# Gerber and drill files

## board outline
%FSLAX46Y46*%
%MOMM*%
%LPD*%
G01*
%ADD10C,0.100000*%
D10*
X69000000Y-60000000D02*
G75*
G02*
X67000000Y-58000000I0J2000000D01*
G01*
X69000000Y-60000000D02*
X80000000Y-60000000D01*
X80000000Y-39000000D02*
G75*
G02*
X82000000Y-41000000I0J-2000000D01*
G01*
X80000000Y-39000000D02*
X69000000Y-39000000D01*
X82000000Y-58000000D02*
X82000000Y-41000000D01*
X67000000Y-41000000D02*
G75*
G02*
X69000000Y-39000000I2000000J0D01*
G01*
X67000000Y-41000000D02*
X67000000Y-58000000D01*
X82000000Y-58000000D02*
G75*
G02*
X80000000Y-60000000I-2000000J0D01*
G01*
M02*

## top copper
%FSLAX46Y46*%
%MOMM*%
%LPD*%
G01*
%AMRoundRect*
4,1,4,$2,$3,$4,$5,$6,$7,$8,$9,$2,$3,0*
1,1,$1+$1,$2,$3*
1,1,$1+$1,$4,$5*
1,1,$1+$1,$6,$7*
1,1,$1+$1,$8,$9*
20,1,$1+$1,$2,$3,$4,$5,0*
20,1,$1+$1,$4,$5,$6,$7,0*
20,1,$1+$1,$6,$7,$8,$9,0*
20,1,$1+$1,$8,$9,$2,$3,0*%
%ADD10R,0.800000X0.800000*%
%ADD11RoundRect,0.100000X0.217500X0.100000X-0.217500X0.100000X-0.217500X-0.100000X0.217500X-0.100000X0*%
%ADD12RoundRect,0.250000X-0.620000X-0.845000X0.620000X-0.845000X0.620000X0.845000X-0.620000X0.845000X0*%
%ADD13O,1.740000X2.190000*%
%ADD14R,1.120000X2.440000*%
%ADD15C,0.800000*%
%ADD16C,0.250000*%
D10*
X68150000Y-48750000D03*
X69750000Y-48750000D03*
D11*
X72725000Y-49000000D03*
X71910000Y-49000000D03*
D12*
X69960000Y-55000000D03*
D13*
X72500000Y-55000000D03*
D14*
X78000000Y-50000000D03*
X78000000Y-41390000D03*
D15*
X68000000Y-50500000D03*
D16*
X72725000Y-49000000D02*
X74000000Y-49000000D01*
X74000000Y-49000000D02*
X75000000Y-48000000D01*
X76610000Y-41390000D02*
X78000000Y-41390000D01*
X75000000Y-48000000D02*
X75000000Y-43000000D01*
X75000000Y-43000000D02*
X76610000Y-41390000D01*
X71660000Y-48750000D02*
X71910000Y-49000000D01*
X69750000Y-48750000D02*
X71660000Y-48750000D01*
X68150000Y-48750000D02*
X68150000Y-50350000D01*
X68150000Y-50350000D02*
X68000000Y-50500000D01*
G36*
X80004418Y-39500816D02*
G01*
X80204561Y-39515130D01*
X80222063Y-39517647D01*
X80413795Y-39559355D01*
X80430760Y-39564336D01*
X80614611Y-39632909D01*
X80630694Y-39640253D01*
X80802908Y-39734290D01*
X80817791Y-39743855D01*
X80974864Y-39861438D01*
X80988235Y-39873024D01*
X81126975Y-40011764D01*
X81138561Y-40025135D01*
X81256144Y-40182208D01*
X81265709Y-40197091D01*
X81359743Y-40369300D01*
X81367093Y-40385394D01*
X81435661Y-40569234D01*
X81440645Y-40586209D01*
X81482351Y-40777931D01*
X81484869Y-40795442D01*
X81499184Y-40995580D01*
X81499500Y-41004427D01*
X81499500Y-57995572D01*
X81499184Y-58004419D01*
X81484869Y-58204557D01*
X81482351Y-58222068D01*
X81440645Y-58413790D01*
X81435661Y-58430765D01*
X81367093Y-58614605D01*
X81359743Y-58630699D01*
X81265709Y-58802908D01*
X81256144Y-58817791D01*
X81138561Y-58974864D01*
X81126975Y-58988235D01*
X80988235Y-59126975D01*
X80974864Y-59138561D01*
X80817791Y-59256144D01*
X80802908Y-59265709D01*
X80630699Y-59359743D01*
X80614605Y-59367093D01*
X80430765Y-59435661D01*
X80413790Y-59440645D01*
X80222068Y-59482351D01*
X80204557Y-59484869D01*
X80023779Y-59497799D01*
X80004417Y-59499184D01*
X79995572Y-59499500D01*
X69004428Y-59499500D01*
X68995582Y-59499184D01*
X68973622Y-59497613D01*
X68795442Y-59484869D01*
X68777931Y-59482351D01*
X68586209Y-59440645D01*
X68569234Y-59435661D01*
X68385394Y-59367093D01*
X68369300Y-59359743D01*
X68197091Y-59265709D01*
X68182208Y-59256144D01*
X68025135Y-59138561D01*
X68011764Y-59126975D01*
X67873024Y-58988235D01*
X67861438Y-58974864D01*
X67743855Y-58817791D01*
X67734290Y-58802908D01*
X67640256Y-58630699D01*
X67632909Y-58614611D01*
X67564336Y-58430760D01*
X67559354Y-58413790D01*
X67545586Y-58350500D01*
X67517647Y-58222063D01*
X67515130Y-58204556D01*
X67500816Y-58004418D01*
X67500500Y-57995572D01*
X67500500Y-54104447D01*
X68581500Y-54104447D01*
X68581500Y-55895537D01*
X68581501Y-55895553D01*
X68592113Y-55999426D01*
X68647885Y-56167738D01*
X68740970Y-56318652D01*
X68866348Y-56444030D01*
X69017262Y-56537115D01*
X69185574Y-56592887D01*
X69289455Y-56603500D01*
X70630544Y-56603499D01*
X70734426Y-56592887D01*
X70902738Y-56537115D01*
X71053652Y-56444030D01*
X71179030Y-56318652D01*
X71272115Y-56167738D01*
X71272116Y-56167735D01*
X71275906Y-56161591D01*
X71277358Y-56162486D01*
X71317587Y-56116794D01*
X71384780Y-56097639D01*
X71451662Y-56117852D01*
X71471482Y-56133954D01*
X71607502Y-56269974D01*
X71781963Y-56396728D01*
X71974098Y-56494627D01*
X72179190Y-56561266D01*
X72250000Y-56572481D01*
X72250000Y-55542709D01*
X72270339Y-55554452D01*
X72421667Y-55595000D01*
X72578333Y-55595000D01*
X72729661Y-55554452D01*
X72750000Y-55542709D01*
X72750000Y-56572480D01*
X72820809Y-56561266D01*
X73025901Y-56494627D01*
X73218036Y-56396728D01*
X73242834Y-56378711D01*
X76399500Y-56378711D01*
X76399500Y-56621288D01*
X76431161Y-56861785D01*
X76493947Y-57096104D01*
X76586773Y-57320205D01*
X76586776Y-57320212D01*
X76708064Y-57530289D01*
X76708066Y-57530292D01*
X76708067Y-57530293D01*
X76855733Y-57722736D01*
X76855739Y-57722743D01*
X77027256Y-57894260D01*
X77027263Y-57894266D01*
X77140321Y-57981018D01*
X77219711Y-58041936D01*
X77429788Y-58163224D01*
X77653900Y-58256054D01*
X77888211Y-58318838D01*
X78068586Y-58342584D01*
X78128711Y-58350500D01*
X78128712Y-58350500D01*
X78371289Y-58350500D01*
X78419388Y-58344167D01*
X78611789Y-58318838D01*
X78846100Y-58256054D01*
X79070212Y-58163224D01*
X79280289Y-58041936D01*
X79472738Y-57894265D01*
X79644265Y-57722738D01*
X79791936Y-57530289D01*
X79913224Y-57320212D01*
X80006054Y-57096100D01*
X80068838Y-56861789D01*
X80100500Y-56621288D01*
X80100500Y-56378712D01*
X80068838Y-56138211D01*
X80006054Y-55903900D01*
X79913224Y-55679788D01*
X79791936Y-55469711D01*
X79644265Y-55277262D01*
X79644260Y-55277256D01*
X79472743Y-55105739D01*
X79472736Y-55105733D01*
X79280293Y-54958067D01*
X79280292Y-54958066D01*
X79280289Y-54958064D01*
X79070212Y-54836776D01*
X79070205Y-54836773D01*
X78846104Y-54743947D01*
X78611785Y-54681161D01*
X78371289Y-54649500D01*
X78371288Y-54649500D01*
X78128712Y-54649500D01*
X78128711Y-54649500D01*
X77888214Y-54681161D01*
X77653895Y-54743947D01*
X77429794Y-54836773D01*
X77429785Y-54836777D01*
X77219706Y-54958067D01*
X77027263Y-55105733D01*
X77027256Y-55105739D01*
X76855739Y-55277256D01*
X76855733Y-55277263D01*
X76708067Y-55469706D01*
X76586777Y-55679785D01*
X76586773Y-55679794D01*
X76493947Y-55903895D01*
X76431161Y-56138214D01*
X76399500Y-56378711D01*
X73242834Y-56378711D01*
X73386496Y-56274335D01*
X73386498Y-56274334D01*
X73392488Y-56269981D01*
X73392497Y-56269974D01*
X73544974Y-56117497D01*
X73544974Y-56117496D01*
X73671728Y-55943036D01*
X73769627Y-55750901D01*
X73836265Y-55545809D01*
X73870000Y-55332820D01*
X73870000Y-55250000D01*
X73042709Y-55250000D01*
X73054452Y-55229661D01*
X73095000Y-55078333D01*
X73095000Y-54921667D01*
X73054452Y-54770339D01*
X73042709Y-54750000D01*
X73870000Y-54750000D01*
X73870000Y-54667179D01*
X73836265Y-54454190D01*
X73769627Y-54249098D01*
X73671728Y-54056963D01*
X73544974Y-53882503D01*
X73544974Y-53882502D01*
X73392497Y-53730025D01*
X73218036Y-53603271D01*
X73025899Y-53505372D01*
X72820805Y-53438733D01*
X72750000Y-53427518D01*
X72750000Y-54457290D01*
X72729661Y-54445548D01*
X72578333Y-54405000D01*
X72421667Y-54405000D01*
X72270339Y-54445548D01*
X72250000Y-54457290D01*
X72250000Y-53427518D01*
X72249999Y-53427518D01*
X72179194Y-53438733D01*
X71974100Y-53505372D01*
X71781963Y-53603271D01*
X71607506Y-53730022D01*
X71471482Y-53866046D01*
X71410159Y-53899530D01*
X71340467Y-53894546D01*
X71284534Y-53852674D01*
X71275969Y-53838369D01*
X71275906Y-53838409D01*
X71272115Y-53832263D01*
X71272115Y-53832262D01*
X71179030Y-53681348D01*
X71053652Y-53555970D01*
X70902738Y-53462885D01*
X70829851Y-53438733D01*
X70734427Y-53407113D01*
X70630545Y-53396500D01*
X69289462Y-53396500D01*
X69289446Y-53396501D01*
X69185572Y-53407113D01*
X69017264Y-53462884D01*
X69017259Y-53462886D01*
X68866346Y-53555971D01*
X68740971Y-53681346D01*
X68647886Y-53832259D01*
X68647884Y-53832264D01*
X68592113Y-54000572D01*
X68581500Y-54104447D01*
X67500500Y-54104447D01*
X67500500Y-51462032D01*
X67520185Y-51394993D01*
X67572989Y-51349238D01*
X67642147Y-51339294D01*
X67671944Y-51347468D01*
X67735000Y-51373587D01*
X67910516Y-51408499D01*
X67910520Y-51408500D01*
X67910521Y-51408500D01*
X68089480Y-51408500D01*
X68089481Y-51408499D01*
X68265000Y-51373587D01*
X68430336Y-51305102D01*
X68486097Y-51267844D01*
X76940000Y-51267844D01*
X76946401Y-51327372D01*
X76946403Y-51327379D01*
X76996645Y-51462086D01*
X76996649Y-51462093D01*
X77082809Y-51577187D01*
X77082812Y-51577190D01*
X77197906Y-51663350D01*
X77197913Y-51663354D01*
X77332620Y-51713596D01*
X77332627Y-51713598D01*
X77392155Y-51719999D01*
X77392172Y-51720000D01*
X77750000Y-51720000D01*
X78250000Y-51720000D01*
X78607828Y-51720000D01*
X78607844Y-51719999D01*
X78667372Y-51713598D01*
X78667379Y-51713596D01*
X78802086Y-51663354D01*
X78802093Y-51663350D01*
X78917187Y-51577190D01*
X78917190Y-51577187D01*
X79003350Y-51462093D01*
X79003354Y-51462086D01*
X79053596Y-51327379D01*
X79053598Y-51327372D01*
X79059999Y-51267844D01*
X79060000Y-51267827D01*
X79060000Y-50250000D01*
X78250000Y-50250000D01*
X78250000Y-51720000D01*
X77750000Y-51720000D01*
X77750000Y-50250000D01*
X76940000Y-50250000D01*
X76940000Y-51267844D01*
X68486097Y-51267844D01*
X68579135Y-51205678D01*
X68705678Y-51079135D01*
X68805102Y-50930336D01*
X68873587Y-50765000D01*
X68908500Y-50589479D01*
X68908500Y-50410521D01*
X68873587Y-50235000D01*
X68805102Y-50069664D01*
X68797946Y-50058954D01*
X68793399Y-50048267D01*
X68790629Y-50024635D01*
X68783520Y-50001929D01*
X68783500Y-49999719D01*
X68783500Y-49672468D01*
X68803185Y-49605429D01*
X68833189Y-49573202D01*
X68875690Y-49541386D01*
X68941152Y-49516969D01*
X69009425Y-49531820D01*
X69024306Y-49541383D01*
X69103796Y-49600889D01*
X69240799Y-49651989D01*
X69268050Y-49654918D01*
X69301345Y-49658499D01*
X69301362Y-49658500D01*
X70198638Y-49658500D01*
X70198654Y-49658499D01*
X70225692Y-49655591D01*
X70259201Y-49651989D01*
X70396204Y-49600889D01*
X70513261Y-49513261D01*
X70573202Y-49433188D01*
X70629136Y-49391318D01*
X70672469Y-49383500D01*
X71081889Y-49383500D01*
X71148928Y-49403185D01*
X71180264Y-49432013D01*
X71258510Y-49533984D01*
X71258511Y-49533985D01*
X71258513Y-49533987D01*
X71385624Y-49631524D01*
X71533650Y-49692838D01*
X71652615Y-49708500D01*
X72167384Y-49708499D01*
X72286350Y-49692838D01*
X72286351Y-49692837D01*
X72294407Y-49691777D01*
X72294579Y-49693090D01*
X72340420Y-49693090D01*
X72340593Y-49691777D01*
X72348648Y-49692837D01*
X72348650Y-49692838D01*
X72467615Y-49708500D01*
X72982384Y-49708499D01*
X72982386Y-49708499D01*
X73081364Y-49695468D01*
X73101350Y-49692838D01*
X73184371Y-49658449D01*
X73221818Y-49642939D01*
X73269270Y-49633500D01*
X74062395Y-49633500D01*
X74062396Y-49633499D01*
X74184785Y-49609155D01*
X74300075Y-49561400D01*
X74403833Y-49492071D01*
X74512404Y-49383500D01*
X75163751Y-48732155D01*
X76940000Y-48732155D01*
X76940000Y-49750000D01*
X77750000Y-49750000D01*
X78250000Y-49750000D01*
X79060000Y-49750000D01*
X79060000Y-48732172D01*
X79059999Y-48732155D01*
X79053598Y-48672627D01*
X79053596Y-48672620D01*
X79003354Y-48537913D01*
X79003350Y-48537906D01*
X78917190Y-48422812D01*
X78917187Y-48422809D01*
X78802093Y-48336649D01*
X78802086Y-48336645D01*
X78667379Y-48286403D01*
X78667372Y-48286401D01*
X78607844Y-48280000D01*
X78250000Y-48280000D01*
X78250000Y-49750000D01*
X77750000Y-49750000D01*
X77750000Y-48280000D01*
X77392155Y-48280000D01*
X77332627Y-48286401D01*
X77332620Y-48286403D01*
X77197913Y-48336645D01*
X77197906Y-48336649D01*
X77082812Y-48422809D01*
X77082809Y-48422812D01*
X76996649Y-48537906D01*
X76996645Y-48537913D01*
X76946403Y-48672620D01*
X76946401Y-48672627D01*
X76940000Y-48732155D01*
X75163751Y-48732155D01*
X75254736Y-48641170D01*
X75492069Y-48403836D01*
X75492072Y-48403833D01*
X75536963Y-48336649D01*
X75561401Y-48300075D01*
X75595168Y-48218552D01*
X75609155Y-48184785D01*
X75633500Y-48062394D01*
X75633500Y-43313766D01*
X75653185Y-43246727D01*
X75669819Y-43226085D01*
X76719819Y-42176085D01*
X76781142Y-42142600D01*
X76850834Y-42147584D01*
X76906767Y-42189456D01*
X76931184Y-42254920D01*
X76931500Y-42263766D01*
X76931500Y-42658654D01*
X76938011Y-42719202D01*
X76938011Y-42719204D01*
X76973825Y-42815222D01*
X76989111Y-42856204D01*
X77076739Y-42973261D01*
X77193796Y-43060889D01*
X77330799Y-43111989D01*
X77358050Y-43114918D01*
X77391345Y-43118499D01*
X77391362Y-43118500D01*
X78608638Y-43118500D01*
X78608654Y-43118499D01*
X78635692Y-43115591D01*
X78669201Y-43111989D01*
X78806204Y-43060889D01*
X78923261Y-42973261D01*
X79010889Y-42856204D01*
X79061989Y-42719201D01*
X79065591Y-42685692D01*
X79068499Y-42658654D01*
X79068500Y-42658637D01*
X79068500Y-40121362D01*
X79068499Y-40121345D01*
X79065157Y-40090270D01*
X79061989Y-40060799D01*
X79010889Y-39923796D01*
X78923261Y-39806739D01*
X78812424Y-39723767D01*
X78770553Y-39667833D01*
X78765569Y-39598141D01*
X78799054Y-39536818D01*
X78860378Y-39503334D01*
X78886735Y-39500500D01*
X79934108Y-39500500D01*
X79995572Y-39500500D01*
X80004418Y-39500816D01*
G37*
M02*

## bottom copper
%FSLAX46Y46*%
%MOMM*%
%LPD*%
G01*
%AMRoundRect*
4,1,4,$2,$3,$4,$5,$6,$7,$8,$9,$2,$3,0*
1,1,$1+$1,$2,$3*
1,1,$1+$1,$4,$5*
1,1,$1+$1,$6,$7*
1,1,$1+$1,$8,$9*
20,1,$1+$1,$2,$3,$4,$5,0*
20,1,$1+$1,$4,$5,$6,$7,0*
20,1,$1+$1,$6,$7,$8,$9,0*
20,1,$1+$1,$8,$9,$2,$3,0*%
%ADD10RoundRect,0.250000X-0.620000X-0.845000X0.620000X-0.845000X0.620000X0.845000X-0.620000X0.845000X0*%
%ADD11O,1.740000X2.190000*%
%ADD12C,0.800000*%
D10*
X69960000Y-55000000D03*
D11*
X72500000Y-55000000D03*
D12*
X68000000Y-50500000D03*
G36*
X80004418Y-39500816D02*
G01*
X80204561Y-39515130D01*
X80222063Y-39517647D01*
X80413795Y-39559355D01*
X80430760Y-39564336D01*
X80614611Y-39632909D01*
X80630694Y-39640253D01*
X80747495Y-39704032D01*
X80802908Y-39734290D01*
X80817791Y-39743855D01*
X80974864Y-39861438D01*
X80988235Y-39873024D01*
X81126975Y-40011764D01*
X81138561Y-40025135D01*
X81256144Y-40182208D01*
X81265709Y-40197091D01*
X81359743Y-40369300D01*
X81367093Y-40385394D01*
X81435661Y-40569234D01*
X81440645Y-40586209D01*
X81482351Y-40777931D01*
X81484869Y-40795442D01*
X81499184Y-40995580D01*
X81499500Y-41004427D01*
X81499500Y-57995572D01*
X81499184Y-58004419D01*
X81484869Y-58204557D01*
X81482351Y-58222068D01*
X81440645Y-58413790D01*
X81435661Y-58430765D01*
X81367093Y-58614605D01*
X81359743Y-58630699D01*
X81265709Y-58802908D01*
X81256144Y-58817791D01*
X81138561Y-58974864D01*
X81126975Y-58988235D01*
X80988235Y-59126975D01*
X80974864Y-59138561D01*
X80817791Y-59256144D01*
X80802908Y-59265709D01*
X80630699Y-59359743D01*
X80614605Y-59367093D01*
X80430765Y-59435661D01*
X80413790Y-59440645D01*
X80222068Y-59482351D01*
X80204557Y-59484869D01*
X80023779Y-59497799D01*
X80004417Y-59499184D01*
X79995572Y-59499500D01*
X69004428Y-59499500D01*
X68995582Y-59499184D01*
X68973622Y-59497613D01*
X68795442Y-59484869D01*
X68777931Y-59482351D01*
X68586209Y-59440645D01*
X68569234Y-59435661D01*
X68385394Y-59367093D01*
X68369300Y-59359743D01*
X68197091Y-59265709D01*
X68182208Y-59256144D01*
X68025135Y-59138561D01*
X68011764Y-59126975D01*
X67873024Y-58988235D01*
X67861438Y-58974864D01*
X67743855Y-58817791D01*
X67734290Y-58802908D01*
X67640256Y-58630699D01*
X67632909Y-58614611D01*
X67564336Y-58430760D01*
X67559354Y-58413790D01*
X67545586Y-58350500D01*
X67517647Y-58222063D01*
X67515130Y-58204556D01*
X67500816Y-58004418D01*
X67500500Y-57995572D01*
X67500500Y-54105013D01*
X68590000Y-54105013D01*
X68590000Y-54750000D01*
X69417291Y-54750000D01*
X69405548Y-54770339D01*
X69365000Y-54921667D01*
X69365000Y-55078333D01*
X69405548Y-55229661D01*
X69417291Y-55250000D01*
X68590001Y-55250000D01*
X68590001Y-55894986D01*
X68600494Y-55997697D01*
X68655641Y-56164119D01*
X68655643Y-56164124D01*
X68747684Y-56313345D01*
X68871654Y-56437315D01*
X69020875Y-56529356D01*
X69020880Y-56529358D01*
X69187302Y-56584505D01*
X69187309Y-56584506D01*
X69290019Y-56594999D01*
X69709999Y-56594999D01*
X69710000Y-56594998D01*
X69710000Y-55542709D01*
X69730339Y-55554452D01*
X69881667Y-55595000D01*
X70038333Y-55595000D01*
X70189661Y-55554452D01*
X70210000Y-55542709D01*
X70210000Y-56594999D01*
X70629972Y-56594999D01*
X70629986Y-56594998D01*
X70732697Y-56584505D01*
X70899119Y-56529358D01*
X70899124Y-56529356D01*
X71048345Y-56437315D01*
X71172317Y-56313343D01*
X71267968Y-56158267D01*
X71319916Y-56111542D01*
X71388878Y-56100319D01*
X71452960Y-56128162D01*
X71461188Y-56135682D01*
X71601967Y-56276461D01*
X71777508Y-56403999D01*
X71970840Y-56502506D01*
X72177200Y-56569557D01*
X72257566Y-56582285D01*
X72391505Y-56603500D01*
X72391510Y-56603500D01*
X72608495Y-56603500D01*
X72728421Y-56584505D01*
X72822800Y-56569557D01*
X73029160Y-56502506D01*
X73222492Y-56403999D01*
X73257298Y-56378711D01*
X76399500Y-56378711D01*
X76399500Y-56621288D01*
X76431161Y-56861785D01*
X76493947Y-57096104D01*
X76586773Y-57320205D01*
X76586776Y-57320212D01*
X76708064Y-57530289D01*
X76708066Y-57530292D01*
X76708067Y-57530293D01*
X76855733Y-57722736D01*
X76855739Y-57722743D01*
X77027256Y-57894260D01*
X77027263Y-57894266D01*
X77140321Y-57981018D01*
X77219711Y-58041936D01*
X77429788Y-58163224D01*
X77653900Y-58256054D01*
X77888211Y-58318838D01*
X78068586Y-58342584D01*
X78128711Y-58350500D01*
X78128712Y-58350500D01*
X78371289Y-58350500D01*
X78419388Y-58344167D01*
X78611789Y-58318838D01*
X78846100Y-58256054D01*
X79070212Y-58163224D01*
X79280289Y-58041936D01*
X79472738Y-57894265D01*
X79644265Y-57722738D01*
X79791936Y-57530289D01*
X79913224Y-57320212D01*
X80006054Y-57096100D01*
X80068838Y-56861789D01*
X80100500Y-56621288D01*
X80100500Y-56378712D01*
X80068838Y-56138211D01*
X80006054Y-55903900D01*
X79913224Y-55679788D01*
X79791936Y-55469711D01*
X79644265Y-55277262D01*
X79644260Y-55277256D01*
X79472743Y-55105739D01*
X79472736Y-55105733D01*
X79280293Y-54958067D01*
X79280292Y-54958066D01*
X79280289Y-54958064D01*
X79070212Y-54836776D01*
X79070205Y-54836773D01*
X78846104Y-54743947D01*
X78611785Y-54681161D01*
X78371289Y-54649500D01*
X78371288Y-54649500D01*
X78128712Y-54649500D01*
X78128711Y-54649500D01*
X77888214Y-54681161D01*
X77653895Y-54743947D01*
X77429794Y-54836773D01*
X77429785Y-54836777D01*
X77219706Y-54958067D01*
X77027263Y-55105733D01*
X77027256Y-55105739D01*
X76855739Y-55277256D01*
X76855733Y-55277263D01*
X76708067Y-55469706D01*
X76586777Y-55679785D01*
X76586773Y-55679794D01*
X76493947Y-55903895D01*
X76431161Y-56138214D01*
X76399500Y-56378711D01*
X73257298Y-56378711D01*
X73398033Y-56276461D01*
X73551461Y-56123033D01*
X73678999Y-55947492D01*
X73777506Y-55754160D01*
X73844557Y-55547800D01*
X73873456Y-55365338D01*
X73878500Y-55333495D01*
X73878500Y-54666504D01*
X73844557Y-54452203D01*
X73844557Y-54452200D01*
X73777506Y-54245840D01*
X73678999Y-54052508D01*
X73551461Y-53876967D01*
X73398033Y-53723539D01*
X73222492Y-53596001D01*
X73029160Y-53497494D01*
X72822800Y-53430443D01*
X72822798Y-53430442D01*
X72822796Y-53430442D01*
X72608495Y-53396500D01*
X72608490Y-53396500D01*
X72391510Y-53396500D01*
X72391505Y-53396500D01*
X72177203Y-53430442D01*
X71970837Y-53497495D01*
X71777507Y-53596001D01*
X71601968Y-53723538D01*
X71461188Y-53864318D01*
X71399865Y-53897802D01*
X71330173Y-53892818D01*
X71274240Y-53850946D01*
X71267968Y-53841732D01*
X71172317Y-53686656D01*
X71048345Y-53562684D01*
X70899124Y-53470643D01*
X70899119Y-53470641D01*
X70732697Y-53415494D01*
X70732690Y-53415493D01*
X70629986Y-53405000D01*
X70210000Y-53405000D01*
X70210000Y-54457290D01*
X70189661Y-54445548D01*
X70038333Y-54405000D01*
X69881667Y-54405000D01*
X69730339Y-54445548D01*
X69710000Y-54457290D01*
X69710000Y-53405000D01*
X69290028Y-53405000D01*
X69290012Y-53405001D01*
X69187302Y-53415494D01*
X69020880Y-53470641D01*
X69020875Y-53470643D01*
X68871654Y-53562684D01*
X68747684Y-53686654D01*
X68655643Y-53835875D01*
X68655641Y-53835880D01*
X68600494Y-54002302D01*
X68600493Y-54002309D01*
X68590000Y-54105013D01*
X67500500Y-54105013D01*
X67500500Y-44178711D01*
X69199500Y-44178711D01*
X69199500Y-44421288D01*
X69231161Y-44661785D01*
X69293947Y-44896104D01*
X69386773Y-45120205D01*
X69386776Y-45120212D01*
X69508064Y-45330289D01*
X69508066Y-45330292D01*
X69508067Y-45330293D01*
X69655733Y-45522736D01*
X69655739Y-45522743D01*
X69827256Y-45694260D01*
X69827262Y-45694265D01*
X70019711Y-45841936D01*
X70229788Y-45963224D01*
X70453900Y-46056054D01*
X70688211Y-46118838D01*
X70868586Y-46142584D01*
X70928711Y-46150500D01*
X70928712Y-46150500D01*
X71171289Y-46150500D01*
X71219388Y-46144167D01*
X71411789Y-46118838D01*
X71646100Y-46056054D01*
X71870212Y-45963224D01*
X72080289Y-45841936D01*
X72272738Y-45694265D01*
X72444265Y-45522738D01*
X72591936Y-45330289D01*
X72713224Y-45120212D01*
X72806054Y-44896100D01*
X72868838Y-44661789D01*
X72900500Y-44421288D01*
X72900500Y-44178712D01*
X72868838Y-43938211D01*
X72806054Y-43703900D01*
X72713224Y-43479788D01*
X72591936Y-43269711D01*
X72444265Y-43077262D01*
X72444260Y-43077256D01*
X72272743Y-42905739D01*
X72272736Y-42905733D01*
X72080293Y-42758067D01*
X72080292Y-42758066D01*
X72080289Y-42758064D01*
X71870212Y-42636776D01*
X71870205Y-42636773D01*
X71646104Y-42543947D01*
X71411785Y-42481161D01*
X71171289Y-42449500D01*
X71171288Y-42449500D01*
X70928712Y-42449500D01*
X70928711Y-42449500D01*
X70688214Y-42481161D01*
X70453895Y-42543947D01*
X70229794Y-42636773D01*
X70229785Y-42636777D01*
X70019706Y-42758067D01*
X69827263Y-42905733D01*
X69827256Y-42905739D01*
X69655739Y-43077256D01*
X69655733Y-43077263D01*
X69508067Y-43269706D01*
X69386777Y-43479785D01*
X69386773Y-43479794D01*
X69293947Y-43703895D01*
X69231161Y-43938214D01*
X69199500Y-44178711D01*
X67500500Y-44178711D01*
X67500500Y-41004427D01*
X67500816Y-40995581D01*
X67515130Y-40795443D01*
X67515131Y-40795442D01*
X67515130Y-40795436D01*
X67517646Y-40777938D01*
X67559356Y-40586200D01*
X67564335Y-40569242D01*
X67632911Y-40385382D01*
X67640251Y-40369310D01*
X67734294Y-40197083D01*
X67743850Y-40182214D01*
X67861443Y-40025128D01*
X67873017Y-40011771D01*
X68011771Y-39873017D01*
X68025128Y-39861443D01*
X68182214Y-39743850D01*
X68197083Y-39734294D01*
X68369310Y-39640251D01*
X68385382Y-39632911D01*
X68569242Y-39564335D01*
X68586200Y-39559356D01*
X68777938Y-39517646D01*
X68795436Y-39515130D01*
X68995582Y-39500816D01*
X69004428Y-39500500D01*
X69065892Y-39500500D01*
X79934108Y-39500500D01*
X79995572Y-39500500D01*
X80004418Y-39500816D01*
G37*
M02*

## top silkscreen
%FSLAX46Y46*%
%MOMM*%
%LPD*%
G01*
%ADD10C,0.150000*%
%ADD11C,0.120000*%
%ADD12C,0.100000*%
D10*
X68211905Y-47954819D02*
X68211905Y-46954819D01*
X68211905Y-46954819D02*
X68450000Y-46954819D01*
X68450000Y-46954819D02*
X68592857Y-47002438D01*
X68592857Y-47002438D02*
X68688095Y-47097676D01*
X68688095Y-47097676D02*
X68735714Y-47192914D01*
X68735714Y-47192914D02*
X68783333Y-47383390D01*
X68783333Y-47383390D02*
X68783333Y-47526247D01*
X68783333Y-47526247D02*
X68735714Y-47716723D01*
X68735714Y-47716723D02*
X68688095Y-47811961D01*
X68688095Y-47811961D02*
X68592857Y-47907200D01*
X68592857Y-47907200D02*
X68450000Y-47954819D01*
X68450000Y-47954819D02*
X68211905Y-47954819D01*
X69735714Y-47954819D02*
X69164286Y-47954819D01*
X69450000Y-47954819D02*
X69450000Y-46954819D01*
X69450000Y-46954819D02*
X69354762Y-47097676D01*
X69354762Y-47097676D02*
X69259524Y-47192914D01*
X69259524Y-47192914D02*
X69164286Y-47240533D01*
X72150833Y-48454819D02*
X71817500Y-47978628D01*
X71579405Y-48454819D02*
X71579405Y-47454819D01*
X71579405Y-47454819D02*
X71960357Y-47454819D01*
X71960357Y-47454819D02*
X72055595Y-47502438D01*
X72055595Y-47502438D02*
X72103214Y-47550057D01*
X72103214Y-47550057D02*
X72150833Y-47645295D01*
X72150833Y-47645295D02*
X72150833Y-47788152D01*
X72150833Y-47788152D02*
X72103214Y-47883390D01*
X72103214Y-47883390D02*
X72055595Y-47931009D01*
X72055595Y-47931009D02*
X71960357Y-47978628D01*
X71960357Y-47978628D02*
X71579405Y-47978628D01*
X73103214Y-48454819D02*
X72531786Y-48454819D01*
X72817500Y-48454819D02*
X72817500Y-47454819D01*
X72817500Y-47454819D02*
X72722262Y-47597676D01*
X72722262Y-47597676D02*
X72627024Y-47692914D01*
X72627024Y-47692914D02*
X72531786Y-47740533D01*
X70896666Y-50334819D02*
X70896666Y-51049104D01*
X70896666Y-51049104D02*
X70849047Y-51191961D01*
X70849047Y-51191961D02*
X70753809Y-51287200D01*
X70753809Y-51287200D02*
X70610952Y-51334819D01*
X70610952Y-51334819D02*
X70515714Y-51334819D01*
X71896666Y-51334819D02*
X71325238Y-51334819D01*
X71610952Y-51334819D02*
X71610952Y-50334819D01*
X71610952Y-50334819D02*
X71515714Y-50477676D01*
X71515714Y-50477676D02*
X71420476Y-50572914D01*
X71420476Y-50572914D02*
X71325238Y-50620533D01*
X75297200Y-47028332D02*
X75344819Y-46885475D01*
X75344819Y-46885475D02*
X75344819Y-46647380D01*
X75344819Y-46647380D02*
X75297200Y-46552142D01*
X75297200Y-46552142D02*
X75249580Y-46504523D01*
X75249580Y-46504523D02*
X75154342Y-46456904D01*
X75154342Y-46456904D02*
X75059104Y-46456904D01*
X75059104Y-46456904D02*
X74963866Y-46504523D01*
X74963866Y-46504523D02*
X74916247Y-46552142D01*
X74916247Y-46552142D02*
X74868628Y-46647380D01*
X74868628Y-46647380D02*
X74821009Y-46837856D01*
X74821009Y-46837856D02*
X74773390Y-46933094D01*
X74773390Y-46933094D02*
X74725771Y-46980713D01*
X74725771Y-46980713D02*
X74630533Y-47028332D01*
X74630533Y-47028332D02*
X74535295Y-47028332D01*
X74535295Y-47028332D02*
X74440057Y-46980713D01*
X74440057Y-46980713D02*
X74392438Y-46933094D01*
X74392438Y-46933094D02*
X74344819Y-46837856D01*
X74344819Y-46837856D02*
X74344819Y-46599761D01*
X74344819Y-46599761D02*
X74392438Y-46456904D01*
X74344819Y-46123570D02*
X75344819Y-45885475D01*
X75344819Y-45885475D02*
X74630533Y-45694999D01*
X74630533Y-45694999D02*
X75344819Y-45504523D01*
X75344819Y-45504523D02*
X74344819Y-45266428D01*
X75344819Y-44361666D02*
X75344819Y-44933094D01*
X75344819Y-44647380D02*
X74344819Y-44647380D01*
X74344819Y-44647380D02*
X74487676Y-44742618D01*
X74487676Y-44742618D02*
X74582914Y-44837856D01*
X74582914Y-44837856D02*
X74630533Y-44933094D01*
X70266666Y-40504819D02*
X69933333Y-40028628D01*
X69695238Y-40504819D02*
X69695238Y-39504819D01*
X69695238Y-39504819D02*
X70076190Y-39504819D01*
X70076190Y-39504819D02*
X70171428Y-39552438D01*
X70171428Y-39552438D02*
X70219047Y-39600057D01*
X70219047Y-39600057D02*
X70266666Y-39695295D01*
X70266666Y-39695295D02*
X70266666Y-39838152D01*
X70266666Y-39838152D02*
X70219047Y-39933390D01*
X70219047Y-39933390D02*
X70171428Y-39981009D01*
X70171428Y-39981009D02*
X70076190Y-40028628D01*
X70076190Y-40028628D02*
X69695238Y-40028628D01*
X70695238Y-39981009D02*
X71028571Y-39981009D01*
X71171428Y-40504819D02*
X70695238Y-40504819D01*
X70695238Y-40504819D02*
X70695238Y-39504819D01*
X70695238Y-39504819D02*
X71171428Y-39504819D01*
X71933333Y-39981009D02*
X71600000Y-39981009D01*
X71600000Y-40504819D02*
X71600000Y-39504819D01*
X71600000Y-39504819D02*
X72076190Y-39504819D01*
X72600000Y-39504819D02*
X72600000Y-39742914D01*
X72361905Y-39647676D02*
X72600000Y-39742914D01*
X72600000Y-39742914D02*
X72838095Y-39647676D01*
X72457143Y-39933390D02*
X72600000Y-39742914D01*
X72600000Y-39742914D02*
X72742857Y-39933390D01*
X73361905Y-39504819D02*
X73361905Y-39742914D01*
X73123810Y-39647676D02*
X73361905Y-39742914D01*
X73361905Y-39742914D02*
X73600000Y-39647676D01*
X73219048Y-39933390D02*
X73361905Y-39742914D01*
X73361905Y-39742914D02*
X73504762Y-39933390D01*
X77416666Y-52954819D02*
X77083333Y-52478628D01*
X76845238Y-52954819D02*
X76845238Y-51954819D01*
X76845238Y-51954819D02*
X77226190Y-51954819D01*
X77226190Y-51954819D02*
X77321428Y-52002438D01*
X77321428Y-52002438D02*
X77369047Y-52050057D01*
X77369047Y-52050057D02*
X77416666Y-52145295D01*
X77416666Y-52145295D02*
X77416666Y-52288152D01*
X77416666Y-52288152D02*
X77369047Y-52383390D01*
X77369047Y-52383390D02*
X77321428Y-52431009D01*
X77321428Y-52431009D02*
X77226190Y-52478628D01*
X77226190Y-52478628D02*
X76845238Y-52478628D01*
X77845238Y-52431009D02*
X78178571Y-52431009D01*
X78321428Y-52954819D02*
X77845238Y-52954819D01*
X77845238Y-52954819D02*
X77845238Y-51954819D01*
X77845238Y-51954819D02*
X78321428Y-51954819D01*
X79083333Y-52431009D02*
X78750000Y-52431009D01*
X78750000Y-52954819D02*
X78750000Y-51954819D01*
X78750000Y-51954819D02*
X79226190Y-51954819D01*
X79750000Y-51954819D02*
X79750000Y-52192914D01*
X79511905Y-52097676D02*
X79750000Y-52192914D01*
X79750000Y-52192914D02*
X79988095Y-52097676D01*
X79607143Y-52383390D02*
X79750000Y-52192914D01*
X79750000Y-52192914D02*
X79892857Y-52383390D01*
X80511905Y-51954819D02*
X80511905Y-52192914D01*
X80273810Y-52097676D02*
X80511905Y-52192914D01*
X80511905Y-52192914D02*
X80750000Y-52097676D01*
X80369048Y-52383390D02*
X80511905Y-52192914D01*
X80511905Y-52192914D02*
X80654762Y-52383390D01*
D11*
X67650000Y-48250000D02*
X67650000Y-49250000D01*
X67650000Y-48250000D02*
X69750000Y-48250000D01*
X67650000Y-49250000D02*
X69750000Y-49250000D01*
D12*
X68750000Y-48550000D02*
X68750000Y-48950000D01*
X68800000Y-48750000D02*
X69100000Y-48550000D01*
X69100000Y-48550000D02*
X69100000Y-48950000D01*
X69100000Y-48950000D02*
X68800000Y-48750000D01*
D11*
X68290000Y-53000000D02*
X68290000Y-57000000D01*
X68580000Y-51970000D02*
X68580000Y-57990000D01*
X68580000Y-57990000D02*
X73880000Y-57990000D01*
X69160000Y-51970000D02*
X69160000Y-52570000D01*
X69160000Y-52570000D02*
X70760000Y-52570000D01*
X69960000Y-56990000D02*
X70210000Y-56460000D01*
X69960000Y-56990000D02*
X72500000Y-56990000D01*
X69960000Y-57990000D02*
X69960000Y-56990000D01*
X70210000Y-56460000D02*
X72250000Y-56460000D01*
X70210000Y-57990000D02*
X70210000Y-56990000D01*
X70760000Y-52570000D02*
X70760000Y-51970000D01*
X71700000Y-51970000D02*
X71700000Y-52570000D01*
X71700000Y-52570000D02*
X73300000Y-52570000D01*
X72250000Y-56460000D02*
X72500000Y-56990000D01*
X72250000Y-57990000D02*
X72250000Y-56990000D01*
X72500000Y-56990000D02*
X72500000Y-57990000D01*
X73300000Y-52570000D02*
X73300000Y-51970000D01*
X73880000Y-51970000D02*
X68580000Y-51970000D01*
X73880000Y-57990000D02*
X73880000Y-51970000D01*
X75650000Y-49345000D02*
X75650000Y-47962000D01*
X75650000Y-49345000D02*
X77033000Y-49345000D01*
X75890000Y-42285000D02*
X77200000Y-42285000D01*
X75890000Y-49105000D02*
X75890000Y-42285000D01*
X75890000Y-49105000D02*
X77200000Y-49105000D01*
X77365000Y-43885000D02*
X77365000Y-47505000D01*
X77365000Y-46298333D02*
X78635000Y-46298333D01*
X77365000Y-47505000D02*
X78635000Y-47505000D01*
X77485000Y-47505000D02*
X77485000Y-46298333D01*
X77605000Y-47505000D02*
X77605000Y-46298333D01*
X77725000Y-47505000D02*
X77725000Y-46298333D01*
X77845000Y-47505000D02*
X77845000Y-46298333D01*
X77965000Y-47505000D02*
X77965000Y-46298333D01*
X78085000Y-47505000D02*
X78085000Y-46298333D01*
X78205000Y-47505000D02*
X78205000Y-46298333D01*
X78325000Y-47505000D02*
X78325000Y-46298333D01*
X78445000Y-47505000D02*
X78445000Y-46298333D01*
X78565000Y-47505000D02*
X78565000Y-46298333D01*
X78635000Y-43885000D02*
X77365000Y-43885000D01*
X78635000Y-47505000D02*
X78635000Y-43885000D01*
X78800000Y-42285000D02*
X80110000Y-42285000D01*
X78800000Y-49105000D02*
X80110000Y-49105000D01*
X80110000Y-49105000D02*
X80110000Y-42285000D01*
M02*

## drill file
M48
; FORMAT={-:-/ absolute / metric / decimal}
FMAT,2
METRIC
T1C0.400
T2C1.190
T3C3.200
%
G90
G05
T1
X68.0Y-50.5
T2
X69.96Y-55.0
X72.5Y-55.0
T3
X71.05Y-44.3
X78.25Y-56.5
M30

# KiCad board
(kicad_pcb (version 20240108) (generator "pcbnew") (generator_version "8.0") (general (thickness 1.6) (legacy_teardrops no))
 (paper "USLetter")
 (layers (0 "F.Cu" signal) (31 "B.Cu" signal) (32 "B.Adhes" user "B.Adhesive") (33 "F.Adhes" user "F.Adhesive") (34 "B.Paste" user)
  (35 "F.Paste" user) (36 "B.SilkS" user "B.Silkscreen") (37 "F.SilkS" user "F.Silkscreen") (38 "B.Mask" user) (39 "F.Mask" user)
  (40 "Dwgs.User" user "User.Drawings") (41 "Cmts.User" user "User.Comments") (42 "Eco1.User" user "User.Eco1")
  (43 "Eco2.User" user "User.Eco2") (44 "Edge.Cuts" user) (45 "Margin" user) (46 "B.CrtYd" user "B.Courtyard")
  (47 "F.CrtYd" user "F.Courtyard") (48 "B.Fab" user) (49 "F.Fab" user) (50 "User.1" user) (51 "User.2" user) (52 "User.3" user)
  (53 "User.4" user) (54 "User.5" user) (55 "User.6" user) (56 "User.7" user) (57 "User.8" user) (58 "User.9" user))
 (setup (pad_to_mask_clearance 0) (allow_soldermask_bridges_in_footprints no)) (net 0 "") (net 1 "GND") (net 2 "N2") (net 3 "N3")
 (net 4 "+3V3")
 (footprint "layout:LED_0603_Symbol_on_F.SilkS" (layer "F.Cu") (at 68.95 48.75)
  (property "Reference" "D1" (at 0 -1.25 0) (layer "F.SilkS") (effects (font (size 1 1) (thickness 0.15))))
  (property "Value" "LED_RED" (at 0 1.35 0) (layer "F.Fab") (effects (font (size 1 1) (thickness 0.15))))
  (fp_line (start -1.3 -0.5) (end -1.3 0.5) (stroke (width 0.12) (type solid)) (layer "F.SilkS"))
  (fp_line (start -1.3 -0.5) (end 0.8 -0.5) (stroke (width 0.12) (type solid)) (layer "F.SilkS"))
  (fp_line (start -1.3 0.5) (end 0.8 0.5) (stroke (width 0.12) (type solid)) (layer "F.SilkS"))
  (fp_line (start -0.2 -0.2) (end -0.2 0.2) (stroke (width 0.1) (type solid)) (layer "F.SilkS"))
  (fp_line (start -0.15 0) (end 0.15 -0.2) (stroke (width 0.1) (type solid)) (layer "F.SilkS"))
  (fp_line (start 0.15 -0.2) (end 0.15 0.2) (stroke (width 0.1) (type solid)) (layer "F.SilkS"))
  (fp_line (start 0.15 0.2) (end -0.15 0) (stroke (width 0.1) (type solid)) (layer "F.SilkS"))
  (pad "1" smd rect (at -0.8 0 180) (size 0.8 0.8) (layers "F.Cu" "F.Paste" "F.Mask") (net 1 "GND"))
  (pad "2" smd rect (at 0.8 0 180) (size 0.8 0.8) (layers "F.Cu" "F.Paste" "F.Mask") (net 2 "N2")))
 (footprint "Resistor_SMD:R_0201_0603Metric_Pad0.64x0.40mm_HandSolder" (layer "F.Cu") (at 72.3175 49 180)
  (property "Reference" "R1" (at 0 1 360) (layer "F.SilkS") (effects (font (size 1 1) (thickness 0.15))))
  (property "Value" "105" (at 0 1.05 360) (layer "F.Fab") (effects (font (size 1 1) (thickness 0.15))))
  (pad "" smd roundrect (at -0.4325 0 180) (size 0.458 0.36) (layers "F.Paste") (roundrect_rratio 0.25))
  (pad "" smd roundrect (at 0.4325 0 180) (size 0.458 0.36) (layers "F.Paste") (roundrect_rratio 0.25))
  (pad "1" smd roundrect (at -0.4075 0 180) (size 0.635 0.4) (layers "F.Cu" "F.Mask") (roundrect_rratio 0.25) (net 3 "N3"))
  (pad "2" smd roundrect (at 0.4075 0 180) (size 0.635 0.4) (layers "F.Cu" "F.Mask") (roundrect_rratio 0.25) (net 2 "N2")))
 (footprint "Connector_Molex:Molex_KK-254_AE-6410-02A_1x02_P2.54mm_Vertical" (layer "F.Cu") (at 69.96 55)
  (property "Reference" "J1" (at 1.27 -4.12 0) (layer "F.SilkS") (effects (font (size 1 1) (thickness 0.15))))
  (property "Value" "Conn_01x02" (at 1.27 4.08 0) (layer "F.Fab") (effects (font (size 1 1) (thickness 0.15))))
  (fp_line (start -1.67 -2) (end -1.67 2) (stroke (width 0.12) (type solid)) (layer "F.SilkS"))
  (fp_line (start -1.38 -3.03) (end -1.38 2.99) (stroke (width 0.12) (type solid)) (layer "F.SilkS"))
  (fp_line (start -1.38 2.99) (end 3.92 2.99) (stroke (width 0.12) (type solid)) (layer "F.SilkS"))
  (fp_line (start -0.8 -3.03) (end -0.8 -2.43) (stroke (width 0.12) (type solid)) (layer "F.SilkS"))
  (fp_line (start -0.8 -2.43) (end 0.8 -2.43) (stroke (width 0.12) (type solid)) (layer "F.SilkS"))
  (fp_line (start 0 1.99) (end 0.25 1.46) (stroke (width 0.12) (type solid)) (layer "F.SilkS"))
  (fp_line (start 0 1.99) (end 2.54 1.99) (stroke (width 0.12) (type solid)) (layer "F.SilkS"))
  (fp_line (start 0 2.99) (end 0 1.99) (stroke (width 0.12) (type solid)) (layer "F.SilkS"))
  (fp_line (start 0.25 1.46) (end 2.29 1.46) (stroke (width 0.12) (type solid)) (layer "F.SilkS"))
  (fp_line (start 0.25 2.99) (end 0.25 1.99) (stroke (width 0.12) (type solid)) (layer "F.SilkS"))
  (fp_line (start 0.8 -2.43) (end 0.8 -3.03) (stroke (width 0.12) (type solid)) (layer "F.SilkS"))
  (fp_line (start 1.74 -3.03) (end 1.74 -2.43) (stroke (width 0.12) (type solid)) (layer "F.SilkS"))
  (fp_line (start 1.74 -2.43) (end 3.34 -2.43) (stroke (width 0.12) (type solid)) (layer "F.SilkS"))
  (fp_line (start 2.29 1.46) (end 2.54 1.99) (stroke (width 0.12) (type solid)) (layer "F.SilkS"))
  (fp_line (start 2.29 2.99) (end 2.29 1.99) (stroke (width 0.12) (type solid)) (layer "F.SilkS"))
  (fp_line (start 2.54 1.99) (end 2.54 2.99) (stroke (width 0.12) (type solid)) (layer "F.SilkS"))
  (fp_line (start 3.34 -2.43) (end 3.34 -3.03) (stroke (width 0.12) (type solid)) (layer "F.SilkS"))
  (fp_line (start 3.92 -3.03) (end -1.38 -3.03) (stroke (width 0.12) (type solid)) (layer "F.SilkS"))
  (fp_line (start 3.92 2.99) (end 3.92 -3.03) (stroke (width 0.12) (type solid)) (layer "F.SilkS"))
  (pad "1" thru_hole roundrect (at 0 0) (size 1.74 2.19) (drill 1.19) (layers "*.Cu" "*.Mask") (remove_unused_layers no)
   (roundrect_rratio 0.143678) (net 1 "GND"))
  (pad "2" thru_hole oval (at 2.54 0) (size 1.74 2.19) (drill 1.19) (layers "*.Cu" "*.Mask") (remove_unused_layers no) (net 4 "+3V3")))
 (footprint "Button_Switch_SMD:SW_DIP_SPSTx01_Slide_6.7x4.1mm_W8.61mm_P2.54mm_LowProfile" (layer "F.Cu") (at 78 45.695 90)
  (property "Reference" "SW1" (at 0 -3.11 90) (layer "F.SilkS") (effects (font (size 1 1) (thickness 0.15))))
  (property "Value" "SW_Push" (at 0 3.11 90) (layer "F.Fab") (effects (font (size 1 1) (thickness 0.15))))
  (fp_line (start -3.65 -2.35) (end -2.267 -2.35) (stroke (width 0.12) (type solid)) (layer "F.SilkS"))
  (fp_line (start -3.65 -2.35) (end -3.65 -0.967) (stroke (width 0.12) (type solid)) (layer "F.SilkS"))
  (fp_line (start 3.41 -2.11) (end 3.41 -0.8) (stroke (width 0.12) (type solid)) (layer "F.SilkS"))
  (fp_line (start -3.41 -2.11) (end 3.41 -2.11) (stroke (width 0.12) (type solid)) (layer "F.SilkS"))
  (fp_line (start -3.41 -2.11) (end -3.41 -0.8) (stroke (width 0.12) (type solid)) (layer "F.SilkS"))
  (fp_line (start 1.81 -0.635) (end -1.81 -0.635) (stroke (width 0.12) (type solid)) (layer "F.SilkS"))
  (fp_line (start -0.603333 -0.635) (end -0.603333 0.635) (stroke (width 0.12) (type solid)) (layer "F.SilkS"))
  (fp_line (start -1.81 -0.635) (end -1.81 0.635) (stroke (width 0.12) (type solid)) (layer "F.SilkS"))
  (fp_line (start -1.81 -0.515) (end -0.603333 -0.515) (stroke (width 0.12) (type solid)) (layer "F.SilkS"))
  (fp_line (start -1.81 -0.395) (end -0.603333 -0.395) (stroke (width 0.12) (type solid)) (layer "F.SilkS"))
  (fp_line (start -1.81 -0.275) (end -0.603333 -0.275) (stroke (width 0.12) (type solid)) (layer "F.SilkS"))
  (fp_line (start -1.81 -0.155) (end -0.603333 -0.155) (stroke (width 0.12) (type solid)) (layer "F.SilkS"))
  (fp_line (start -1.81 -0.035) (end -0.603333 -0.035) (stroke (width 0.12) (type solid)) (layer "F.SilkS"))
  (fp_line (start -1.81 0.085) (end -0.603333 0.085) (stroke (width 0.12) (type solid)) (layer "F.SilkS"))
  (fp_line (start -1.81 0.205) (end -0.603333 0.205) (stroke (width 0.12) (type solid)) (layer "F.SilkS"))
  (fp_line (start -1.81 0.325) (end -0.603333 0.325) (stroke (width 0.12) (type solid)) (layer "F.SilkS"))
  (fp_line (start -1.81 0.445) (end -0.603333 0.445) (stroke (width 0.12) (type solid)) (layer "F.SilkS"))
  (fp_line (start -1.81 0.565) (end -0.603333 0.565) (stroke (width 0.12) (type solid)) (layer "F.SilkS"))
  (fp_line (start 1.81 0.635) (end 1.81 -0.635) (stroke (width 0.12) (type solid)) (layer "F.SilkS"))
  (fp_line (start -1.81 0.635) (end 1.81 0.635) (stroke (width 0.12) (type solid)) (layer "F.SilkS"))
  (fp_line (start 3.41 0.8) (end 3.41 2.11) (stroke (width 0.12) (type solid)) (layer "F.SilkS"))
  (fp_line (start -3.41 0.8) (end -3.41 2.11) (stroke (width 0.12) (type solid)) (layer "F.SilkS"))
  (fp_line (start -3.41 2.11) (end 3.41 2.11) (stroke (width 0.12) (type solid)) (layer "F.SilkS"))
  (pad "1" smd rect (at -4.305 0 90) (size 2.44 1.12) (layers "F.Cu" "F.Paste" "F.Mask") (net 4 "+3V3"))
  (pad "2" smd rect (at 4.305 0 90) (size 2.44 1.12) (layers "F.Cu" "F.Paste" "F.Mask") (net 3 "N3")))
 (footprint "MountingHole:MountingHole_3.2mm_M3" (layer "F.Cu") (at 71.05 44.3)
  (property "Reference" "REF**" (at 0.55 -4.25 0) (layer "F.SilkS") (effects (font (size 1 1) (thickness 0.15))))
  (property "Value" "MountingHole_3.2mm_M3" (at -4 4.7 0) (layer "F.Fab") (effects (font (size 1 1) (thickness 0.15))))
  (pad "" np_thru_hole circle (at 0 0) (size 3.2 3.2) (drill 3.2) (layers "*.Cu" "*.Mask")))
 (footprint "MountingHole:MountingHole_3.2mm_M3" (layer "F.Cu") (at 78.25 56.5)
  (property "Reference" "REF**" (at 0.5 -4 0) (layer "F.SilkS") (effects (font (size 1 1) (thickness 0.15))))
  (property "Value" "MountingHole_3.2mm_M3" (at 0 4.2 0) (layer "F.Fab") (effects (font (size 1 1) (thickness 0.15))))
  (pad "" np_thru_hole circle (at 0 0) (size 3.2 3.2) (drill 3.2) (layers "*.Cu" "*.Mask")))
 (gr_arc (start 69 60) (mid 67.585786 59.414214) (end 67 58) (stroke (width 0.1) (type default)) (layer "Edge.Cuts"))
 (gr_line (start 69 60) (end 80 60) (stroke (width 0.1) (type default)) (layer "Edge.Cuts"))
 (gr_arc (start 80 39) (mid 81.414214 39.585786) (end 82 41) (stroke (width 0.1) (type default)) (layer "Edge.Cuts"))
 (gr_line (start 80 39) (end 69 39) (stroke (width 0.1) (type default)) (layer "Edge.Cuts"))
 (gr_line (start 82 58) (end 82 41) (stroke (width 0.1) (type default)) (layer "Edge.Cuts"))
 (gr_arc (start 67 41) (mid 67.585786 39.585786) (end 69 39) (stroke (width 0.1) (type default)) (layer "Edge.Cuts"))
 (gr_line (start 67 41) (end 67 58) (stroke (width 0.1) (type default)) (layer "Edge.Cuts"))
 (gr_arc (start 82 58) (mid 81.414214 59.414214) (end 80 60) (stroke (width 0.1) (type default)) (layer "Edge.Cuts"))
 (segment (start 72.725 49) (end 74 49) (width 0.25) (layer "F.Cu") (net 3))
 (segment (start 74 49) (end 75 48) (width 0.25) (layer "F.Cu") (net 3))
 (segment (start 76.61 41.39) (end 78 41.39) (width 0.25) (layer "F.Cu") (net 3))
 (segment (start 75 48) (end 75 43) (width 0.25) (layer "F.Cu") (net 3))
 (segment (start 75 43) (end 76.61 41.39) (width 0.25) (layer "F.Cu") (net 3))
 (segment (start 71.66 48.75) (end 71.91 49) (width 0.25) (layer "F.Cu") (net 2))
 (segment (start 69.75 48.75) (end 71.66 48.75) (width 0.25) (layer "F.Cu") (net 2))
 (segment (start 68.15 48.75) (end 68.15 50.35) (width 0.25) (layer "F.Cu") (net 1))
 (segment (start 68.15 50.35) (end 68 50.5) (width 0.25) (layer "F.Cu") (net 1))
 (via (at 68 50.5) (size 0.8) (drill 0.4) (layers "F.Cu" "B.Cu") (free yes) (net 1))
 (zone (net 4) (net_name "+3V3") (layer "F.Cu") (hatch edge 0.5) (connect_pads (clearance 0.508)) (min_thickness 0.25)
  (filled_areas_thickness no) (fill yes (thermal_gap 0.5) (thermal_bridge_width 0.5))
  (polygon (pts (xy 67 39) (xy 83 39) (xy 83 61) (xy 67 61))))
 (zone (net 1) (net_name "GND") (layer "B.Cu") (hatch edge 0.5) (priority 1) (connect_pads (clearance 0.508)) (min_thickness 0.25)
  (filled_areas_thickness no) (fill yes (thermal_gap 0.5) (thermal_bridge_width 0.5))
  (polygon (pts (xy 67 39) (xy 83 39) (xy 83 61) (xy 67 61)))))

